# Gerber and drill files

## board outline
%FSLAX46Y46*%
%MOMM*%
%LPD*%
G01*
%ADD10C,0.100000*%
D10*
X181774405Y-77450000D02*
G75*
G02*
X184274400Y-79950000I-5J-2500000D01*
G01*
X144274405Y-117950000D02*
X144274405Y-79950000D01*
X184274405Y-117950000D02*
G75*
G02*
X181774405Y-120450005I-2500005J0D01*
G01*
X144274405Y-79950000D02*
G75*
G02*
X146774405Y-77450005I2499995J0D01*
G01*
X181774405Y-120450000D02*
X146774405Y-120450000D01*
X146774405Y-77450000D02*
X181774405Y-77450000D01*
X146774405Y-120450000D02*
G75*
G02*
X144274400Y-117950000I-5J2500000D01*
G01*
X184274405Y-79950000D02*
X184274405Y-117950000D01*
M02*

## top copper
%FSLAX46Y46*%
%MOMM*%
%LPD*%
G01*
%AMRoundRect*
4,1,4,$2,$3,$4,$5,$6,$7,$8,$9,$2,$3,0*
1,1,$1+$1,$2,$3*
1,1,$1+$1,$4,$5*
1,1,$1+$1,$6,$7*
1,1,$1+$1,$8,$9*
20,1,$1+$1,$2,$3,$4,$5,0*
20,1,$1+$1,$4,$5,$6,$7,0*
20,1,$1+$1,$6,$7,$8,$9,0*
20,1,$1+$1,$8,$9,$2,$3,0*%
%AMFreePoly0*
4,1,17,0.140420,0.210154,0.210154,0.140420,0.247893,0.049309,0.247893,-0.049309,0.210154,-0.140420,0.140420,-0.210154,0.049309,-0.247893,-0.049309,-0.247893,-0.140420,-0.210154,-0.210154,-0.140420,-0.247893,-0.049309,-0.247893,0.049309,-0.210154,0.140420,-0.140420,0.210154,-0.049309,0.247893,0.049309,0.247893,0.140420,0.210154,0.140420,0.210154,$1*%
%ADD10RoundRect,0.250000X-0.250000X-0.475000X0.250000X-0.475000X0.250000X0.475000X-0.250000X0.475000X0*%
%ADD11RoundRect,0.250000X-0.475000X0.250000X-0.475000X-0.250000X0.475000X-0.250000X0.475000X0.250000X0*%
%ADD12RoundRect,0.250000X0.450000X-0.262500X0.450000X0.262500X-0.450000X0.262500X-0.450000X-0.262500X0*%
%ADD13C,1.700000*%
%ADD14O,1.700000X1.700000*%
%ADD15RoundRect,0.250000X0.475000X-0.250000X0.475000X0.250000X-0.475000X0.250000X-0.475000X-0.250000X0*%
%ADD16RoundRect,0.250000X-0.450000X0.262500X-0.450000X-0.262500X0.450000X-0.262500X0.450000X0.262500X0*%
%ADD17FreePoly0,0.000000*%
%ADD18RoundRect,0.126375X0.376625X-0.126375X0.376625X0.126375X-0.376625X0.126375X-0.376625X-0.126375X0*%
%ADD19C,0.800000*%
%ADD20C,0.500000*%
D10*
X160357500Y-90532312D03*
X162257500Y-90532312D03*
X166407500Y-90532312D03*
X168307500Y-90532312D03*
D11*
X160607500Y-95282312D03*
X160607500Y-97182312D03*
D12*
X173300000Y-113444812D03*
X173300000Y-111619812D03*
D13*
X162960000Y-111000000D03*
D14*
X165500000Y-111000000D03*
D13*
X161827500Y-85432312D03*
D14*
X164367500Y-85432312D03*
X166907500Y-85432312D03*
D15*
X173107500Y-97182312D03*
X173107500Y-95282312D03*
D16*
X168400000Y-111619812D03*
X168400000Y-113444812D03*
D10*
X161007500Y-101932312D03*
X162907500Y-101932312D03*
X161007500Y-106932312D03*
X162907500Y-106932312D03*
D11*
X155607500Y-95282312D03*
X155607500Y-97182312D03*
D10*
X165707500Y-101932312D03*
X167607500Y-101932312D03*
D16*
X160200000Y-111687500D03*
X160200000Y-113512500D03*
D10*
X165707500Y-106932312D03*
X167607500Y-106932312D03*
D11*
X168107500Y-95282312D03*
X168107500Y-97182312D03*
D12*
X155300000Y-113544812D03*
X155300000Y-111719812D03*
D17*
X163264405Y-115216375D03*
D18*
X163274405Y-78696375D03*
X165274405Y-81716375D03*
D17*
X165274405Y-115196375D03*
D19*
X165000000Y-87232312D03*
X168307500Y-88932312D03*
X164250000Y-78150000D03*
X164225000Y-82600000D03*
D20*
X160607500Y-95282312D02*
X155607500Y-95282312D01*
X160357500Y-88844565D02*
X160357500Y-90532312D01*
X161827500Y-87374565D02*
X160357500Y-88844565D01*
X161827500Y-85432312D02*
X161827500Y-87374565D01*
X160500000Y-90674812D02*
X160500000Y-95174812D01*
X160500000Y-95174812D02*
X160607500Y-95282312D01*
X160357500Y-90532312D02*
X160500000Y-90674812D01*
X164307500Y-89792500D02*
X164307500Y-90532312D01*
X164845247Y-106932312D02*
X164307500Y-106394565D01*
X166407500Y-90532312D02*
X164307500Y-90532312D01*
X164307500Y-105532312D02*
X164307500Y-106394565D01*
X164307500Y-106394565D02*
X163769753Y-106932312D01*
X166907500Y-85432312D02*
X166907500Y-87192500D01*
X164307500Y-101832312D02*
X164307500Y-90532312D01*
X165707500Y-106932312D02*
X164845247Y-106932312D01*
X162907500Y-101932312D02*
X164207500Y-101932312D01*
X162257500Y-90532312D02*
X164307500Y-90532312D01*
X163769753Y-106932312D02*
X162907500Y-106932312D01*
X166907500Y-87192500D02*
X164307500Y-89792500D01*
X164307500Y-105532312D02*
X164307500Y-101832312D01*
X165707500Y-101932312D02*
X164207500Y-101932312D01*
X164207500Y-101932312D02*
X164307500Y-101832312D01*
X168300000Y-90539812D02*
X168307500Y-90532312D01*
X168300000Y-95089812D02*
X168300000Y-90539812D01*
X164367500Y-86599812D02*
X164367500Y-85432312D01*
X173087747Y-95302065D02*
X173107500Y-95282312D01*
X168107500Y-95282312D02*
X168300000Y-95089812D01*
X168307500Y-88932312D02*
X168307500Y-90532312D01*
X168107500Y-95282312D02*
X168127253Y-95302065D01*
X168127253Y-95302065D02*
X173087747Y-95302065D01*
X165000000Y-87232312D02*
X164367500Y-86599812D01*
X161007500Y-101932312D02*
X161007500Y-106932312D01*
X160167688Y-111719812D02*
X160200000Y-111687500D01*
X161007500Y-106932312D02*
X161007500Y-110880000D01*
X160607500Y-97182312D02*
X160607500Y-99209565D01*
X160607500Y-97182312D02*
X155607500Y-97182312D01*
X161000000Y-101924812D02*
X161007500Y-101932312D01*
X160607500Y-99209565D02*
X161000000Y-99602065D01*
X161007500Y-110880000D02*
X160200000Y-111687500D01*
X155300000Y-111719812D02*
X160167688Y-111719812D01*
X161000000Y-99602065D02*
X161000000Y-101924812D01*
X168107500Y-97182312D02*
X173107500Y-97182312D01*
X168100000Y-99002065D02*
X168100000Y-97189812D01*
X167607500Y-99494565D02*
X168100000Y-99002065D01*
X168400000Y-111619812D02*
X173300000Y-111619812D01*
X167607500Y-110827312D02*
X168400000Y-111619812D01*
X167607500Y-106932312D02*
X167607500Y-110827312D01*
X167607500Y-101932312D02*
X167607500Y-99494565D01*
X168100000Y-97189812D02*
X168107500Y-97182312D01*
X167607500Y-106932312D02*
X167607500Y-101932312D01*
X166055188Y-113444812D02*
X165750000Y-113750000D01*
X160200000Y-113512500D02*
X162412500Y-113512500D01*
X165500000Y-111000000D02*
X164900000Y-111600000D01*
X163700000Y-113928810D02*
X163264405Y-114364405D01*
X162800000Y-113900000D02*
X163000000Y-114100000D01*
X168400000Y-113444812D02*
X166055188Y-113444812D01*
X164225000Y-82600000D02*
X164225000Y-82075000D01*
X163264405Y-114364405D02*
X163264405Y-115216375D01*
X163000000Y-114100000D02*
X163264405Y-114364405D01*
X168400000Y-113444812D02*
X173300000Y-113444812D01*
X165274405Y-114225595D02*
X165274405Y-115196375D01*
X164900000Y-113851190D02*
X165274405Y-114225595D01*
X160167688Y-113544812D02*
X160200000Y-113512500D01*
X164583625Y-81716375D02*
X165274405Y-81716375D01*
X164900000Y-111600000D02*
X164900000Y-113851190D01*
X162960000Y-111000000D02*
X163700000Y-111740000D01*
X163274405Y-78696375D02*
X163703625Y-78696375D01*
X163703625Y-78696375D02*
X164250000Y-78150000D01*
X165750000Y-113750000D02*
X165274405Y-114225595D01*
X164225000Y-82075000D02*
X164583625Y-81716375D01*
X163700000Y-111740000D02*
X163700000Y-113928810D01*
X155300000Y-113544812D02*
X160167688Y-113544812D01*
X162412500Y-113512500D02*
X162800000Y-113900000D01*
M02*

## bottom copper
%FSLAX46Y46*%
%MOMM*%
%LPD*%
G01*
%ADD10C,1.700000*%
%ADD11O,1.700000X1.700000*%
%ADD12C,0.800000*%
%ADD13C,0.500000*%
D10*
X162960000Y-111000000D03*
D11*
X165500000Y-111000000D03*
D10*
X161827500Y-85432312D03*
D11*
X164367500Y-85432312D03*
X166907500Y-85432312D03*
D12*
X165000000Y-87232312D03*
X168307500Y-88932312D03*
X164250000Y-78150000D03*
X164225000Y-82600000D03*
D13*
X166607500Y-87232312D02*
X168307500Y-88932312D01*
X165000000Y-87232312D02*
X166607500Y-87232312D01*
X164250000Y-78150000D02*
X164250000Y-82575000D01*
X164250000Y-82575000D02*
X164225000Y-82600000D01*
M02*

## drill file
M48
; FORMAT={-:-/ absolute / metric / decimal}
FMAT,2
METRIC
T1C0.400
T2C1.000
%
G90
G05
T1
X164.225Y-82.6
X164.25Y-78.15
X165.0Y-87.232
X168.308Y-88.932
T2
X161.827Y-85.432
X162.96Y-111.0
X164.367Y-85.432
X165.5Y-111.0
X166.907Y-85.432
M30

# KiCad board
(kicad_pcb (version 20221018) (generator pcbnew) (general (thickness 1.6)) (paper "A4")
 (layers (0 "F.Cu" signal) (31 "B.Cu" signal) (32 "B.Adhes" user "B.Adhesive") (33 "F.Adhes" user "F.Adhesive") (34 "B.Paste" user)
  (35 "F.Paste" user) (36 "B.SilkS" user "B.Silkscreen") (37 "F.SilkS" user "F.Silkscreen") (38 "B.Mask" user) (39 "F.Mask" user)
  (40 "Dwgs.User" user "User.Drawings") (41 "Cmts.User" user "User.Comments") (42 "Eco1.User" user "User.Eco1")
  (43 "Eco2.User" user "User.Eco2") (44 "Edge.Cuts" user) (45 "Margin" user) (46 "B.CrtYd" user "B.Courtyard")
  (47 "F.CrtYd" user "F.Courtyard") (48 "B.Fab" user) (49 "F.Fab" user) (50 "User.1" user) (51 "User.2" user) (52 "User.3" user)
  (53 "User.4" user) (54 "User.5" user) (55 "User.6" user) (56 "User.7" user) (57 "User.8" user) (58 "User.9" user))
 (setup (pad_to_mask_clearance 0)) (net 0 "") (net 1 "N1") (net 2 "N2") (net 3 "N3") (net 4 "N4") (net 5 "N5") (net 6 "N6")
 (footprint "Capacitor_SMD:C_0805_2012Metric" (layer "F.Cu") (at 161.3075 90.532312)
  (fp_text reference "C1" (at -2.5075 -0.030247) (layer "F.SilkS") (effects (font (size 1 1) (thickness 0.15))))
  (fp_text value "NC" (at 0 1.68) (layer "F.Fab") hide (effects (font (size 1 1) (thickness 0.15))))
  (pad "1" smd roundrect (at -0.95 0) (size 1 1.45) (layers "F.Cu" "F.Paste" "F.Mask") (roundrect_rratio 0.25) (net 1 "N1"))
  (pad "2" smd roundrect (at 0.95 0) (size 1 1.45) (layers "F.Cu" "F.Paste" "F.Mask") (roundrect_rratio 0.25) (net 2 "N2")))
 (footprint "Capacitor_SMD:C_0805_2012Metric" (layer "F.Cu") (at 167.3575 90.532312)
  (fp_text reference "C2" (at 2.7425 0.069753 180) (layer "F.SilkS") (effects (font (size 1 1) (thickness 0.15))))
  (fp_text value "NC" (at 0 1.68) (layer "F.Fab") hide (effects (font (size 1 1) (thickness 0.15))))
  (pad "1" smd roundrect (at -0.95 0) (size 1 1.45) (layers "F.Cu" "F.Paste" "F.Mask") (roundrect_rratio 0.25) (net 2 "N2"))
  (pad "2" smd roundrect (at 0.95 0) (size 1 1.45) (layers "F.Cu" "F.Paste" "F.Mask") (roundrect_rratio 0.25) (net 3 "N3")))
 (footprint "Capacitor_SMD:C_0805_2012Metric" (layer "F.Cu") (at 160.6075 96.232312 -90)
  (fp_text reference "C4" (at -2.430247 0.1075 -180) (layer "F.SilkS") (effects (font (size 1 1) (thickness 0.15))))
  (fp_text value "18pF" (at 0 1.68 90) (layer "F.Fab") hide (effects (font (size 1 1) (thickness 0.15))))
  (pad "1" smd roundrect (at -0.95 0 270) (size 1 1.45) (layers "F.Cu" "F.Paste" "F.Mask") (roundrect_rratio 0.25) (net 1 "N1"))
  (pad "2" smd roundrect (at 0.95 0 270) (size 1 1.45) (layers "F.Cu" "F.Paste" "F.Mask") (roundrect_rratio 0.25) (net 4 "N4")))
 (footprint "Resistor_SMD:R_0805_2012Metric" (layer "F.Cu") (at 173.3 112.532312 90)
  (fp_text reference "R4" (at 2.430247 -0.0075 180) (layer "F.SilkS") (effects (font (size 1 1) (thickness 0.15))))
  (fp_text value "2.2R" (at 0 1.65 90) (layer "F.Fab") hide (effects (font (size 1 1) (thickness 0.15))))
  (pad "1" smd roundrect (at -0.9125 0 90) (size 1.025 1.4) (layers "F.Cu" "F.Paste" "F.Mask") (roundrect_rratio 0.243902) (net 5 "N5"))
  (pad "2" smd roundrect (at 0.9125 0 90) (size 1.025 1.4) (layers "F.Cu" "F.Paste" "F.Mask") (roundrect_rratio 0.243902) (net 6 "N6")))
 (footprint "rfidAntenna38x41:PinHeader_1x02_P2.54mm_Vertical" (layer "F.Cu") (at 162.96 111 90)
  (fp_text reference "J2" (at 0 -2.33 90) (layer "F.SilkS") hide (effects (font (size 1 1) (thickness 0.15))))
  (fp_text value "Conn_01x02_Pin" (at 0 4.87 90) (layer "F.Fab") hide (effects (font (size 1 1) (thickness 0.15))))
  (pad "1" thru_hole circle (at 0 0 90) (size 1.7 1.7) (drill 1) (layers "*.Cu" "*.Mask") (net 5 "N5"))
  (pad "2" thru_hole oval (at 0 2.54 90) (size 1.7 1.7) (drill 1) (layers "*.Cu" "*.Mask") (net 5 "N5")))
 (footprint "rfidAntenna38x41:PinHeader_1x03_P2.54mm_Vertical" (layer "F.Cu") (at 161.8275 85.432312 90)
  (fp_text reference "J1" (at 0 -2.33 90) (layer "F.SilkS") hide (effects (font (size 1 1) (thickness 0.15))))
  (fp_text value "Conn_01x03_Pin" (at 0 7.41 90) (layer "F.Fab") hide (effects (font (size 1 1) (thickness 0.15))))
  (pad "1" thru_hole circle (at 0 0 90) (size 1.7 1.7) (drill 1) (layers "*.Cu" "*.Mask") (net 1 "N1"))
  (pad "2" thru_hole oval (at 0 2.54 90) (size 1.7 1.7) (drill 1) (layers "*.Cu" "*.Mask") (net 3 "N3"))
  (pad "3" thru_hole oval (at 0 5.08 90) (size 1.7 1.7) (drill 1) (layers "*.Cu" "*.Mask") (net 2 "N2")))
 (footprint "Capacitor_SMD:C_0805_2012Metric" (layer "F.Cu") (at 173.1075 96.232312 90)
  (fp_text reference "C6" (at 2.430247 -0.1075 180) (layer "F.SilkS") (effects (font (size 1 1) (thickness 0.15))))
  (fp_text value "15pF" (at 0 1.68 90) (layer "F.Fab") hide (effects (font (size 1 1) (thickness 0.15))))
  (pad "1" smd roundrect (at -0.95 0 90) (size 1 1.45) (layers "F.Cu" "F.Paste" "F.Mask") (roundrect_rratio 0.25) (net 6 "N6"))
  (pad "2" smd roundrect (at 0.95 0 90) (size 1 1.45) (layers "F.Cu" "F.Paste" "F.Mask") (roundrect_rratio 0.25) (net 3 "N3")))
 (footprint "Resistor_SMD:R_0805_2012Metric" (layer "F.Cu") (at 168.4 112.532312 -90)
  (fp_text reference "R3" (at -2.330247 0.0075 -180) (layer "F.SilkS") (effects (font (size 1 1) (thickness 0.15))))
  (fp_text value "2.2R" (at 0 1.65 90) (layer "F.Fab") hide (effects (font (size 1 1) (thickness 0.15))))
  (pad "1" smd roundrect (at -0.9125 0 270) (size 1.025 1.4) (layers "F.Cu" "F.Paste" "F.Mask") (roundrect_rratio 0.243902) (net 6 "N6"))
  (pad "2" smd roundrect (at 0.9125 0 270) (size 1.025 1.4) (layers "F.Cu" "F.Paste" "F.Mask") (roundrect_rratio 0.243902) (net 5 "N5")))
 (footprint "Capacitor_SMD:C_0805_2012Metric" (layer "F.Cu") (at 161.9575 101.932312)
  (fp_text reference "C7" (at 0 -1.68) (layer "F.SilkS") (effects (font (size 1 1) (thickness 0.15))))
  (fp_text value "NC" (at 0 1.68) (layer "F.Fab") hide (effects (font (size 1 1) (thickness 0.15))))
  (pad "1" smd roundrect (at -0.95 0) (size 1 1.45) (layers "F.Cu" "F.Paste" "F.Mask") (roundrect_rratio 0.25) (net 4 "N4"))
  (pad "2" smd roundrect (at 0.95 0) (size 1 1.45) (layers "F.Cu" "F.Paste" "F.Mask") (roundrect_rratio 0.25) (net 2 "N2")))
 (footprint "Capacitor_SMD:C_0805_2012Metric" (layer "F.Cu") (at 161.9575 106.932312)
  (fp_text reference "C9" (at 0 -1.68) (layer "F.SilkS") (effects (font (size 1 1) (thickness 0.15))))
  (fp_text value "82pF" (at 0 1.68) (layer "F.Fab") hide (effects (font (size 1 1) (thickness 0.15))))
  (pad "1" smd roundrect (at -0.95 0) (size 1 1.45) (layers "F.Cu" "F.Paste" "F.Mask") (roundrect_rratio 0.25) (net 4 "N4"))
  (pad "2" smd roundrect (at 0.95 0) (size 1 1.45) (layers "F.Cu" "F.Paste" "F.Mask") (roundrect_rratio 0.25) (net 2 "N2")))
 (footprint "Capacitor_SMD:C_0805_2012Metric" (layer "F.Cu") (at 155.6075 96.232312 -90)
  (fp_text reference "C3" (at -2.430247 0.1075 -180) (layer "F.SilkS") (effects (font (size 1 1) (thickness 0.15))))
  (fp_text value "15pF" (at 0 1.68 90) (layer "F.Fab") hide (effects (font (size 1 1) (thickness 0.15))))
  (pad "1" smd roundrect (at -0.95 0 270) (size 1 1.45) (layers "F.Cu" "F.Paste" "F.Mask") (roundrect_rratio 0.25) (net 1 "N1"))
  (pad "2" smd roundrect (at 0.95 0 270) (size 1 1.45) (layers "F.Cu" "F.Paste" "F.Mask") (roundrect_rratio 0.25) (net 4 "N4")))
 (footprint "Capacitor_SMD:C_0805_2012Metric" (layer "F.Cu") (at 166.6575 101.932312)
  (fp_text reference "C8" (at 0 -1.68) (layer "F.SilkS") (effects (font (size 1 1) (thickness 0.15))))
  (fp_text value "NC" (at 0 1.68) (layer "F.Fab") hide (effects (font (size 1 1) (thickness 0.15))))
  (pad "1" smd roundrect (at -0.95 0) (size 1 1.45) (layers "F.Cu" "F.Paste" "F.Mask") (roundrect_rratio 0.25) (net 2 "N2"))
  (pad "2" smd roundrect (at 0.95 0) (size 1 1.45) (layers "F.Cu" "F.Paste" "F.Mask") (roundrect_rratio 0.25) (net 6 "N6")))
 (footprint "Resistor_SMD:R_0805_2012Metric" (layer "F.Cu") (at 160.2 112.6 -90)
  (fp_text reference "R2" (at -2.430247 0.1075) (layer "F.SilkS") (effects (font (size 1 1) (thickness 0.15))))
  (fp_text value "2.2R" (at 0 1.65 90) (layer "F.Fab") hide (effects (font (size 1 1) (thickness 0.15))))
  (pad "1" smd roundrect (at -0.9125 0 270) (size 1.025 1.4) (layers "F.Cu" "F.Paste" "F.Mask") (roundrect_rratio 0.243902) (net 4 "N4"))
  (pad "2" smd roundrect (at 0.9125 0 270) (size 1.025 1.4) (layers "F.Cu" "F.Paste" "F.Mask") (roundrect_rratio 0.243902) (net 5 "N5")))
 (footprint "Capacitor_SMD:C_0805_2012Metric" (layer "F.Cu") (at 166.6575 106.932312)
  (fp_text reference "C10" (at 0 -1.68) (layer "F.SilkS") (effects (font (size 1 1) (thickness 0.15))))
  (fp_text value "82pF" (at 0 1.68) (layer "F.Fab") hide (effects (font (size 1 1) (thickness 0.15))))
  (pad "1" smd roundrect (at -0.95 0) (size 1 1.45) (layers "F.Cu" "F.Paste" "F.Mask") (roundrect_rratio 0.25) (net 2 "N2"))
  (pad "2" smd roundrect (at 0.95 0) (size 1 1.45) (layers "F.Cu" "F.Paste" "F.Mask") (roundrect_rratio 0.25) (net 6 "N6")))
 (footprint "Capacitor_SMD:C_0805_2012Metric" (layer "F.Cu") (at 168.1075 96.232312 -90)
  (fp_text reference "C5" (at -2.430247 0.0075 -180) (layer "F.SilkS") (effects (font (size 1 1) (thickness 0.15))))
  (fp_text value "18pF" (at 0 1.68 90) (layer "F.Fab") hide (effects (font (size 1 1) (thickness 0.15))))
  (pad "1" smd roundrect (at -0.95 0 270) (size 1 1.45) (layers "F.Cu" "F.Paste" "F.Mask") (roundrect_rratio 0.25) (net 3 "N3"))
  (pad "2" smd roundrect (at 0.95 0 270) (size 1 1.45) (layers "F.Cu" "F.Paste" "F.Mask") (roundrect_rratio 0.25) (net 6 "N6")))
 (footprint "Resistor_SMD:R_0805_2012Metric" (layer "F.Cu") (at 155.3 112.632312 90)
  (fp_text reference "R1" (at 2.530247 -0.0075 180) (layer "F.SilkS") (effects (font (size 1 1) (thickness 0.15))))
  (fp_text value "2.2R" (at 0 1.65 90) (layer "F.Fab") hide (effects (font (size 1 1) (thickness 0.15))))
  (pad "1" smd roundrect (at -0.9125 0 90) (size 1.025 1.4) (layers "F.Cu" "F.Paste" "F.Mask") (roundrect_rratio 0.243902) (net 5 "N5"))
  (pad "2" smd roundrect (at 0.9125 0 90) (size 1.025 1.4) (layers "F.Cu" "F.Paste" "F.Mask") (roundrect_rratio 0.243902) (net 4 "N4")))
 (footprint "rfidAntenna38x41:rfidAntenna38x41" (layer "F.Cu") (at 145.524405 78.706375)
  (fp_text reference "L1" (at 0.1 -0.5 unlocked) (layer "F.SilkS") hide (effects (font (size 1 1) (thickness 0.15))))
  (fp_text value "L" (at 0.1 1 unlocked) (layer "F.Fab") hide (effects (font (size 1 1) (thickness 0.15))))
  (pad "1" smd custom (at 17.74 36.51) (size 0.5055 0.5055) (layers "F.Cu" "F.Paste") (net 5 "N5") (thermal_bridge_angle 45)
   (options (clearance outline) (anchor circle)) (primitives))
  (pad "1" smd roundrect (at 17.75 -0.01 90) (size 0.5055 1.006) (layers "F.Cu" "F.Paste") (roundrect_rratio 0.25) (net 5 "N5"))
  (pad "2" smd roundrect (at 19.75 3.01 90) (size 0.5055 1.006) (layers "F.Cu" "F.Paste") (roundrect_rratio 0.25) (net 5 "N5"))
  (pad "2" smd custom (at 19.75 36.49) (size 0.5055 0.5055) (layers "F.Cu" "F.Paste") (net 5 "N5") (thermal_bridge_angle 45)
   (options (clearance outline) (anchor circle)) (primitives)))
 (gr_arc (start 181.774405 77.45) (mid 183.542169 78.182235) (end 184.274405 79.95) (stroke (width 0.1) (type default)) (layer "Edge.Cuts"))
 (gr_line (start 144.274405 117.95) (end 144.274405 79.95) (stroke (width 0.1) (type default)) (layer "Edge.Cuts"))
 (gr_arc (start 184.274405 117.95) (mid 183.542172 119.717767) (end 181.774405 120.45) (stroke (width 0.1) (type default))
  (layer "Edge.Cuts"))
 (gr_arc (start 144.274405 79.95) (mid 145.006638 78.182233) (end 146.774405 77.45) (stroke (width 0.1) (type default)) (layer "Edge.Cuts"))
 (gr_line (start 181.774405 120.45) (end 146.774405 120.45) (stroke (width 0.1) (type default)) (layer "Edge.Cuts"))
 (gr_line (start 146.774405 77.45) (end 181.774405 77.45) (stroke (width 0.1) (type default)) (layer "Edge.Cuts"))
 (gr_arc (start 146.774405 120.45) (mid 145.006638 119.717767) (end 144.274405 117.95) (stroke (width 0.1) (type default))
  (layer "Edge.Cuts"))
 (gr_line (start 184.274405 79.95) (end 184.274405 117.95) (stroke (width 0.1) (type default)) (layer "Edge.Cuts"))
 (segment (start 160.6075 95.282312) (end 155.6075 95.282312) (width 0.5) (layer "F.Cu") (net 1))
 (segment (start 160.3575 88.844565) (end 160.3575 90.532312) (width 0.5) (layer "F.Cu") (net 1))
 (segment (start 161.8275 87.374565) (end 160.3575 88.844565) (width 0.5) (layer "F.Cu") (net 1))
 (segment (start 161.8275 85.432312) (end 161.8275 87.374565) (width 0.5) (layer "F.Cu") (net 1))
 (segment (start 160.5 90.674812) (end 160.5 95.174812) (width 0.5) (layer "F.Cu") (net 1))
 (segment (start 160.5 95.174812) (end 160.6075 95.282312) (width 0.5) (layer "F.Cu") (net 1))
 (segment (start 160.3575 90.532312) (end 160.5 90.674812) (width 0.5) (layer "F.Cu") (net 1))
 (segment (start 164.3075 89.7925) (end 164.3075 90.532312) (width 0.5) (layer "F.Cu") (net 2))
 (segment (start 164.845247 106.932312) (end 164.3075 106.394565) (width 0.5) (layer "F.Cu") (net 2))
 (segment (start 166.4075 90.532312) (end 164.3075 90.532312) (width 0.5) (layer "F.Cu") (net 2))
 (segment (start 164.3075 105.532312) (end 164.3075 106.394565) (width 0.5) (layer "F.Cu") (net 2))
 (segment (start 164.3075 106.394565) (end 163.769753 106.932312) (width 0.5) (layer "F.Cu") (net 2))
 (segment (start 166.9075 85.432312) (end 166.9075 87.1925) (width 0.5) (layer "F.Cu") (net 2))
 (segment (start 164.3075 101.832312) (end 164.3075 90.532312) (width 0.5) (layer "F.Cu") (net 2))
 (segment (start 165.7075 106.932312) (end 164.845247 106.932312) (width 0.5) (layer "F.Cu") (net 2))
 (segment (start 162.9075 101.932312) (end 164.2075 101.932312) (width 0.5) (layer "F.Cu") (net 2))
 (segment (start 162.2575 90.532312) (end 164.3075 90.532312) (width 0.5) (layer "F.Cu") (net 2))
 (segment (start 163.769753 106.932312) (end 162.9075 106.932312) (width 0.5) (layer "F.Cu") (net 2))
 (segment (start 166.9075 87.1925) (end 164.3075 89.7925) (width 0.5) (layer "F.Cu") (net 2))
 (segment (start 164.3075 105.532312) (end 164.3075 101.832312) (width 0.5) (layer "F.Cu") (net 2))
 (segment (start 165.7075 101.932312) (end 164.2075 101.932312) (width 0.5) (layer "F.Cu") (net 2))
 (segment (start 164.2075 101.932312) (end 164.3075 101.832312) (width 0.5) (layer "F.Cu") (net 2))
 (segment (start 168.3 90.539812) (end 168.3075 90.532312) (width 0.5) (layer "F.Cu") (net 3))
 (segment (start 168.3 95.089812) (end 168.3 90.539812) (width 0.5) (layer "F.Cu") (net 3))
 (segment (start 164.3675 86.599812) (end 164.3675 85.432312) (width 0.5) (layer "F.Cu") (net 3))
 (segment (start 173.087747 95.302065) (end 173.1075 95.282312) (width 0.5) (layer "F.Cu") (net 3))
 (segment (start 168.1075 95.282312) (end 168.3 95.089812) (width 0.5) (layer "F.Cu") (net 3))
 (segment (start 168.3075 88.932312) (end 168.3075 90.532312) (width 0.5) (layer "F.Cu") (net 3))
 (segment (start 168.1075 95.282312) (end 168.127253 95.302065) (width 0.5) (layer "F.Cu") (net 3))
 (segment (start 168.127253 95.302065) (end 173.087747 95.302065) (width 0.5) (layer "F.Cu") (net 3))
 (segment (start 165 87.232312) (end 164.3675 86.599812) (width 0.5) (layer "F.Cu") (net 3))
 (via (at 165 87.232312) (size 0.8) (drill 0.4) (layers "F.Cu" "B.Cu") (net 3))
 (via (at 168.3075 88.932312) (size 0.8) (drill 0.4) (layers "F.Cu" "B.Cu") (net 3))
 (segment (start 166.6075 87.232312) (end 168.3075 88.932312) (width 0.5) (layer "B.Cu") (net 3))
 (segment (start 165 87.232312) (end 166.6075 87.232312) (width 0.5) (layer "B.Cu") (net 3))
 (segment (start 161.0075 101.932312) (end 161.0075 106.932312) (width 0.5) (layer "F.Cu") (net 4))
 (segment (start 160.167688 111.719812) (end 160.2 111.6875) (width 0.5) (layer "F.Cu") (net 4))
 (segment (start 161.0075 106.932312) (end 161.0075 110.88) (width 0.5) (layer "F.Cu") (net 4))
 (segment (start 160.6075 97.182312) (end 160.6075 99.209565) (width 0.5) (layer "F.Cu") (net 4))
 (segment (start 160.6075 97.182312) (end 155.6075 97.182312) (width 0.5) (layer "F.Cu") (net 4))
 (segment (start 161 101.924812) (end 161.0075 101.932312) (width 0.5) (layer "F.Cu") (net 4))
 (segment (start 160.6075 99.209565) (end 161 99.602065) (width 0.5) (layer "F.Cu") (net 4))
 (segment (start 161.0075 110.88) (end 160.2 111.6875) (width 0.5) (layer "F.Cu") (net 4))
 (segment (start 155.3 111.719812) (end 160.167688 111.719812) (width 0.5) (layer "F.Cu") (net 4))
 (segment (start 161 99.602065) (end 161 101.924812) (width 0.5) (layer "F.Cu") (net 4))
 (segment (start 168.1075 97.182312) (end 173.1075 97.182312) (width 0.5) (layer "F.Cu") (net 6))
 (segment (start 168.1 99.002065) (end 168.1 97.189812) (width 0.5) (layer "F.Cu") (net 6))
 (segment (start 167.6075 99.494565) (end 168.1 99.002065) (width 0.5) (layer "F.Cu") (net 6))
 (segment (start 168.4 111.619812) (end 173.3 111.619812) (width 0.5) (layer "F.Cu") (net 6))
 (segment (start 167.6075 110.827312) (end 168.4 111.619812) (width 0.5) (layer "F.Cu") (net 6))
 (segment (start 167.6075 106.932312) (end 167.6075 110.827312) (width 0.5) (layer "F.Cu") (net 6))
 (segment (start 167.6075 101.932312) (end 167.6075 99.494565) (width 0.5) (layer "F.Cu") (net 6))
 (segment (start 168.1 97.189812) (end 168.1075 97.182312) (width 0.5) (layer "F.Cu") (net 6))
 (segment (start 167.6075 106.932312) (end 167.6075 101.932312) (width 0.5) (layer "F.Cu") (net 6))
 (segment (start 166.055188 113.444812) (end 165.75 113.75) (width 0.5) (layer "F.Cu") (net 5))
 (segment (start 160.2 113.5125) (end 162.4125 113.5125) (width 0.5) (layer "F.Cu") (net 5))
 (segment (start 165.5 111) (end 164.9 111.6) (width 0.5) (layer "F.Cu") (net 5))
 (segment (start 163.7 113.92881) (end 163.264405 114.364405) (width 0.5) (layer "F.Cu") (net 5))
 (segment (start 162.8 113.9) (end 163 114.1) (width 0.5) (layer "F.Cu") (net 5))
 (segment (start 168.4 113.444812) (end 166.055188 113.444812) (width 0.5) (layer "F.Cu") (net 5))
 (segment (start 164.225 82.6) (end 164.225 82.075) (width 0.5) (layer "F.Cu") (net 5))
 (segment (start 163.264405 114.364405) (end 163.264405 115.216375) (width 0.5) (layer "F.Cu") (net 5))
 (segment (start 163 114.1) (end 163.264405 114.364405) (width 0.5) (layer "F.Cu") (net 5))
 (segment (start 168.4 113.444812) (end 173.3 113.444812) (width 0.5) (layer "F.Cu") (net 5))
 (segment (start 165.274405 114.225595) (end 165.274405 115.196375) (width 0.5) (layer "F.Cu") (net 5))
 (segment (start 164.9 113.85119) (end 165.274405 114.225595) (width 0.5) (layer "F.Cu") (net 5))
 (segment (start 160.167688 113.544812) (end 160.2 113.5125) (width 0.5) (layer "F.Cu") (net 5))
 (segment (start 164.583625 81.716375) (end 165.274405 81.716375) (width 0.5) (layer "F.Cu") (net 5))
 (segment (start 164.9 111.6) (end 164.9 113.85119) (width 0.5) (layer "F.Cu") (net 5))
 (segment (start 162.96 111) (end 163.7 111.74) (width 0.5) (layer "F.Cu") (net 5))
 (segment (start 163.274405 78.696375) (end 163.703625 78.696375) (width 0.5) (layer "F.Cu") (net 5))
 (segment (start 163.703625 78.696375) (end 164.25 78.15) (width 0.5) (layer "F.Cu") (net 5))
 (segment (start 165.75 113.75) (end 165.274405 114.225595) (width 0.5) (layer "F.Cu") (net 5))
 (segment (start 164.225 82.075) (end 164.583625 81.716375) (width 0.5) (layer "F.Cu") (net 5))
 (segment (start 163.7 111.74) (end 163.7 113.92881) (width 0.5) (layer "F.Cu") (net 5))
 (segment (start 155.3 113.544812) (end 160.167688 113.544812) (width 0.5) (layer "F.Cu") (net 5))
 (segment (start 162.4125 113.5125) (end 162.8 113.9) (width 0.5) (layer "F.Cu") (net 5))
 (via (at 164.25 78.15) (size 0.8) (drill 0.4) (layers "F.Cu" "B.Cu") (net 5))
 (via (at 164.225 82.6) (size 0.8) (drill 0.4) (layers "F.Cu" "B.Cu") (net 5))
 (segment (start 164.25 78.15) (end 164.25 82.575) (width 0.5) (layer "B.Cu") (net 5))
 (segment (start 164.25 82.575) (end 164.225 82.6) (width 0.5) (layer "B.Cu") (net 5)))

